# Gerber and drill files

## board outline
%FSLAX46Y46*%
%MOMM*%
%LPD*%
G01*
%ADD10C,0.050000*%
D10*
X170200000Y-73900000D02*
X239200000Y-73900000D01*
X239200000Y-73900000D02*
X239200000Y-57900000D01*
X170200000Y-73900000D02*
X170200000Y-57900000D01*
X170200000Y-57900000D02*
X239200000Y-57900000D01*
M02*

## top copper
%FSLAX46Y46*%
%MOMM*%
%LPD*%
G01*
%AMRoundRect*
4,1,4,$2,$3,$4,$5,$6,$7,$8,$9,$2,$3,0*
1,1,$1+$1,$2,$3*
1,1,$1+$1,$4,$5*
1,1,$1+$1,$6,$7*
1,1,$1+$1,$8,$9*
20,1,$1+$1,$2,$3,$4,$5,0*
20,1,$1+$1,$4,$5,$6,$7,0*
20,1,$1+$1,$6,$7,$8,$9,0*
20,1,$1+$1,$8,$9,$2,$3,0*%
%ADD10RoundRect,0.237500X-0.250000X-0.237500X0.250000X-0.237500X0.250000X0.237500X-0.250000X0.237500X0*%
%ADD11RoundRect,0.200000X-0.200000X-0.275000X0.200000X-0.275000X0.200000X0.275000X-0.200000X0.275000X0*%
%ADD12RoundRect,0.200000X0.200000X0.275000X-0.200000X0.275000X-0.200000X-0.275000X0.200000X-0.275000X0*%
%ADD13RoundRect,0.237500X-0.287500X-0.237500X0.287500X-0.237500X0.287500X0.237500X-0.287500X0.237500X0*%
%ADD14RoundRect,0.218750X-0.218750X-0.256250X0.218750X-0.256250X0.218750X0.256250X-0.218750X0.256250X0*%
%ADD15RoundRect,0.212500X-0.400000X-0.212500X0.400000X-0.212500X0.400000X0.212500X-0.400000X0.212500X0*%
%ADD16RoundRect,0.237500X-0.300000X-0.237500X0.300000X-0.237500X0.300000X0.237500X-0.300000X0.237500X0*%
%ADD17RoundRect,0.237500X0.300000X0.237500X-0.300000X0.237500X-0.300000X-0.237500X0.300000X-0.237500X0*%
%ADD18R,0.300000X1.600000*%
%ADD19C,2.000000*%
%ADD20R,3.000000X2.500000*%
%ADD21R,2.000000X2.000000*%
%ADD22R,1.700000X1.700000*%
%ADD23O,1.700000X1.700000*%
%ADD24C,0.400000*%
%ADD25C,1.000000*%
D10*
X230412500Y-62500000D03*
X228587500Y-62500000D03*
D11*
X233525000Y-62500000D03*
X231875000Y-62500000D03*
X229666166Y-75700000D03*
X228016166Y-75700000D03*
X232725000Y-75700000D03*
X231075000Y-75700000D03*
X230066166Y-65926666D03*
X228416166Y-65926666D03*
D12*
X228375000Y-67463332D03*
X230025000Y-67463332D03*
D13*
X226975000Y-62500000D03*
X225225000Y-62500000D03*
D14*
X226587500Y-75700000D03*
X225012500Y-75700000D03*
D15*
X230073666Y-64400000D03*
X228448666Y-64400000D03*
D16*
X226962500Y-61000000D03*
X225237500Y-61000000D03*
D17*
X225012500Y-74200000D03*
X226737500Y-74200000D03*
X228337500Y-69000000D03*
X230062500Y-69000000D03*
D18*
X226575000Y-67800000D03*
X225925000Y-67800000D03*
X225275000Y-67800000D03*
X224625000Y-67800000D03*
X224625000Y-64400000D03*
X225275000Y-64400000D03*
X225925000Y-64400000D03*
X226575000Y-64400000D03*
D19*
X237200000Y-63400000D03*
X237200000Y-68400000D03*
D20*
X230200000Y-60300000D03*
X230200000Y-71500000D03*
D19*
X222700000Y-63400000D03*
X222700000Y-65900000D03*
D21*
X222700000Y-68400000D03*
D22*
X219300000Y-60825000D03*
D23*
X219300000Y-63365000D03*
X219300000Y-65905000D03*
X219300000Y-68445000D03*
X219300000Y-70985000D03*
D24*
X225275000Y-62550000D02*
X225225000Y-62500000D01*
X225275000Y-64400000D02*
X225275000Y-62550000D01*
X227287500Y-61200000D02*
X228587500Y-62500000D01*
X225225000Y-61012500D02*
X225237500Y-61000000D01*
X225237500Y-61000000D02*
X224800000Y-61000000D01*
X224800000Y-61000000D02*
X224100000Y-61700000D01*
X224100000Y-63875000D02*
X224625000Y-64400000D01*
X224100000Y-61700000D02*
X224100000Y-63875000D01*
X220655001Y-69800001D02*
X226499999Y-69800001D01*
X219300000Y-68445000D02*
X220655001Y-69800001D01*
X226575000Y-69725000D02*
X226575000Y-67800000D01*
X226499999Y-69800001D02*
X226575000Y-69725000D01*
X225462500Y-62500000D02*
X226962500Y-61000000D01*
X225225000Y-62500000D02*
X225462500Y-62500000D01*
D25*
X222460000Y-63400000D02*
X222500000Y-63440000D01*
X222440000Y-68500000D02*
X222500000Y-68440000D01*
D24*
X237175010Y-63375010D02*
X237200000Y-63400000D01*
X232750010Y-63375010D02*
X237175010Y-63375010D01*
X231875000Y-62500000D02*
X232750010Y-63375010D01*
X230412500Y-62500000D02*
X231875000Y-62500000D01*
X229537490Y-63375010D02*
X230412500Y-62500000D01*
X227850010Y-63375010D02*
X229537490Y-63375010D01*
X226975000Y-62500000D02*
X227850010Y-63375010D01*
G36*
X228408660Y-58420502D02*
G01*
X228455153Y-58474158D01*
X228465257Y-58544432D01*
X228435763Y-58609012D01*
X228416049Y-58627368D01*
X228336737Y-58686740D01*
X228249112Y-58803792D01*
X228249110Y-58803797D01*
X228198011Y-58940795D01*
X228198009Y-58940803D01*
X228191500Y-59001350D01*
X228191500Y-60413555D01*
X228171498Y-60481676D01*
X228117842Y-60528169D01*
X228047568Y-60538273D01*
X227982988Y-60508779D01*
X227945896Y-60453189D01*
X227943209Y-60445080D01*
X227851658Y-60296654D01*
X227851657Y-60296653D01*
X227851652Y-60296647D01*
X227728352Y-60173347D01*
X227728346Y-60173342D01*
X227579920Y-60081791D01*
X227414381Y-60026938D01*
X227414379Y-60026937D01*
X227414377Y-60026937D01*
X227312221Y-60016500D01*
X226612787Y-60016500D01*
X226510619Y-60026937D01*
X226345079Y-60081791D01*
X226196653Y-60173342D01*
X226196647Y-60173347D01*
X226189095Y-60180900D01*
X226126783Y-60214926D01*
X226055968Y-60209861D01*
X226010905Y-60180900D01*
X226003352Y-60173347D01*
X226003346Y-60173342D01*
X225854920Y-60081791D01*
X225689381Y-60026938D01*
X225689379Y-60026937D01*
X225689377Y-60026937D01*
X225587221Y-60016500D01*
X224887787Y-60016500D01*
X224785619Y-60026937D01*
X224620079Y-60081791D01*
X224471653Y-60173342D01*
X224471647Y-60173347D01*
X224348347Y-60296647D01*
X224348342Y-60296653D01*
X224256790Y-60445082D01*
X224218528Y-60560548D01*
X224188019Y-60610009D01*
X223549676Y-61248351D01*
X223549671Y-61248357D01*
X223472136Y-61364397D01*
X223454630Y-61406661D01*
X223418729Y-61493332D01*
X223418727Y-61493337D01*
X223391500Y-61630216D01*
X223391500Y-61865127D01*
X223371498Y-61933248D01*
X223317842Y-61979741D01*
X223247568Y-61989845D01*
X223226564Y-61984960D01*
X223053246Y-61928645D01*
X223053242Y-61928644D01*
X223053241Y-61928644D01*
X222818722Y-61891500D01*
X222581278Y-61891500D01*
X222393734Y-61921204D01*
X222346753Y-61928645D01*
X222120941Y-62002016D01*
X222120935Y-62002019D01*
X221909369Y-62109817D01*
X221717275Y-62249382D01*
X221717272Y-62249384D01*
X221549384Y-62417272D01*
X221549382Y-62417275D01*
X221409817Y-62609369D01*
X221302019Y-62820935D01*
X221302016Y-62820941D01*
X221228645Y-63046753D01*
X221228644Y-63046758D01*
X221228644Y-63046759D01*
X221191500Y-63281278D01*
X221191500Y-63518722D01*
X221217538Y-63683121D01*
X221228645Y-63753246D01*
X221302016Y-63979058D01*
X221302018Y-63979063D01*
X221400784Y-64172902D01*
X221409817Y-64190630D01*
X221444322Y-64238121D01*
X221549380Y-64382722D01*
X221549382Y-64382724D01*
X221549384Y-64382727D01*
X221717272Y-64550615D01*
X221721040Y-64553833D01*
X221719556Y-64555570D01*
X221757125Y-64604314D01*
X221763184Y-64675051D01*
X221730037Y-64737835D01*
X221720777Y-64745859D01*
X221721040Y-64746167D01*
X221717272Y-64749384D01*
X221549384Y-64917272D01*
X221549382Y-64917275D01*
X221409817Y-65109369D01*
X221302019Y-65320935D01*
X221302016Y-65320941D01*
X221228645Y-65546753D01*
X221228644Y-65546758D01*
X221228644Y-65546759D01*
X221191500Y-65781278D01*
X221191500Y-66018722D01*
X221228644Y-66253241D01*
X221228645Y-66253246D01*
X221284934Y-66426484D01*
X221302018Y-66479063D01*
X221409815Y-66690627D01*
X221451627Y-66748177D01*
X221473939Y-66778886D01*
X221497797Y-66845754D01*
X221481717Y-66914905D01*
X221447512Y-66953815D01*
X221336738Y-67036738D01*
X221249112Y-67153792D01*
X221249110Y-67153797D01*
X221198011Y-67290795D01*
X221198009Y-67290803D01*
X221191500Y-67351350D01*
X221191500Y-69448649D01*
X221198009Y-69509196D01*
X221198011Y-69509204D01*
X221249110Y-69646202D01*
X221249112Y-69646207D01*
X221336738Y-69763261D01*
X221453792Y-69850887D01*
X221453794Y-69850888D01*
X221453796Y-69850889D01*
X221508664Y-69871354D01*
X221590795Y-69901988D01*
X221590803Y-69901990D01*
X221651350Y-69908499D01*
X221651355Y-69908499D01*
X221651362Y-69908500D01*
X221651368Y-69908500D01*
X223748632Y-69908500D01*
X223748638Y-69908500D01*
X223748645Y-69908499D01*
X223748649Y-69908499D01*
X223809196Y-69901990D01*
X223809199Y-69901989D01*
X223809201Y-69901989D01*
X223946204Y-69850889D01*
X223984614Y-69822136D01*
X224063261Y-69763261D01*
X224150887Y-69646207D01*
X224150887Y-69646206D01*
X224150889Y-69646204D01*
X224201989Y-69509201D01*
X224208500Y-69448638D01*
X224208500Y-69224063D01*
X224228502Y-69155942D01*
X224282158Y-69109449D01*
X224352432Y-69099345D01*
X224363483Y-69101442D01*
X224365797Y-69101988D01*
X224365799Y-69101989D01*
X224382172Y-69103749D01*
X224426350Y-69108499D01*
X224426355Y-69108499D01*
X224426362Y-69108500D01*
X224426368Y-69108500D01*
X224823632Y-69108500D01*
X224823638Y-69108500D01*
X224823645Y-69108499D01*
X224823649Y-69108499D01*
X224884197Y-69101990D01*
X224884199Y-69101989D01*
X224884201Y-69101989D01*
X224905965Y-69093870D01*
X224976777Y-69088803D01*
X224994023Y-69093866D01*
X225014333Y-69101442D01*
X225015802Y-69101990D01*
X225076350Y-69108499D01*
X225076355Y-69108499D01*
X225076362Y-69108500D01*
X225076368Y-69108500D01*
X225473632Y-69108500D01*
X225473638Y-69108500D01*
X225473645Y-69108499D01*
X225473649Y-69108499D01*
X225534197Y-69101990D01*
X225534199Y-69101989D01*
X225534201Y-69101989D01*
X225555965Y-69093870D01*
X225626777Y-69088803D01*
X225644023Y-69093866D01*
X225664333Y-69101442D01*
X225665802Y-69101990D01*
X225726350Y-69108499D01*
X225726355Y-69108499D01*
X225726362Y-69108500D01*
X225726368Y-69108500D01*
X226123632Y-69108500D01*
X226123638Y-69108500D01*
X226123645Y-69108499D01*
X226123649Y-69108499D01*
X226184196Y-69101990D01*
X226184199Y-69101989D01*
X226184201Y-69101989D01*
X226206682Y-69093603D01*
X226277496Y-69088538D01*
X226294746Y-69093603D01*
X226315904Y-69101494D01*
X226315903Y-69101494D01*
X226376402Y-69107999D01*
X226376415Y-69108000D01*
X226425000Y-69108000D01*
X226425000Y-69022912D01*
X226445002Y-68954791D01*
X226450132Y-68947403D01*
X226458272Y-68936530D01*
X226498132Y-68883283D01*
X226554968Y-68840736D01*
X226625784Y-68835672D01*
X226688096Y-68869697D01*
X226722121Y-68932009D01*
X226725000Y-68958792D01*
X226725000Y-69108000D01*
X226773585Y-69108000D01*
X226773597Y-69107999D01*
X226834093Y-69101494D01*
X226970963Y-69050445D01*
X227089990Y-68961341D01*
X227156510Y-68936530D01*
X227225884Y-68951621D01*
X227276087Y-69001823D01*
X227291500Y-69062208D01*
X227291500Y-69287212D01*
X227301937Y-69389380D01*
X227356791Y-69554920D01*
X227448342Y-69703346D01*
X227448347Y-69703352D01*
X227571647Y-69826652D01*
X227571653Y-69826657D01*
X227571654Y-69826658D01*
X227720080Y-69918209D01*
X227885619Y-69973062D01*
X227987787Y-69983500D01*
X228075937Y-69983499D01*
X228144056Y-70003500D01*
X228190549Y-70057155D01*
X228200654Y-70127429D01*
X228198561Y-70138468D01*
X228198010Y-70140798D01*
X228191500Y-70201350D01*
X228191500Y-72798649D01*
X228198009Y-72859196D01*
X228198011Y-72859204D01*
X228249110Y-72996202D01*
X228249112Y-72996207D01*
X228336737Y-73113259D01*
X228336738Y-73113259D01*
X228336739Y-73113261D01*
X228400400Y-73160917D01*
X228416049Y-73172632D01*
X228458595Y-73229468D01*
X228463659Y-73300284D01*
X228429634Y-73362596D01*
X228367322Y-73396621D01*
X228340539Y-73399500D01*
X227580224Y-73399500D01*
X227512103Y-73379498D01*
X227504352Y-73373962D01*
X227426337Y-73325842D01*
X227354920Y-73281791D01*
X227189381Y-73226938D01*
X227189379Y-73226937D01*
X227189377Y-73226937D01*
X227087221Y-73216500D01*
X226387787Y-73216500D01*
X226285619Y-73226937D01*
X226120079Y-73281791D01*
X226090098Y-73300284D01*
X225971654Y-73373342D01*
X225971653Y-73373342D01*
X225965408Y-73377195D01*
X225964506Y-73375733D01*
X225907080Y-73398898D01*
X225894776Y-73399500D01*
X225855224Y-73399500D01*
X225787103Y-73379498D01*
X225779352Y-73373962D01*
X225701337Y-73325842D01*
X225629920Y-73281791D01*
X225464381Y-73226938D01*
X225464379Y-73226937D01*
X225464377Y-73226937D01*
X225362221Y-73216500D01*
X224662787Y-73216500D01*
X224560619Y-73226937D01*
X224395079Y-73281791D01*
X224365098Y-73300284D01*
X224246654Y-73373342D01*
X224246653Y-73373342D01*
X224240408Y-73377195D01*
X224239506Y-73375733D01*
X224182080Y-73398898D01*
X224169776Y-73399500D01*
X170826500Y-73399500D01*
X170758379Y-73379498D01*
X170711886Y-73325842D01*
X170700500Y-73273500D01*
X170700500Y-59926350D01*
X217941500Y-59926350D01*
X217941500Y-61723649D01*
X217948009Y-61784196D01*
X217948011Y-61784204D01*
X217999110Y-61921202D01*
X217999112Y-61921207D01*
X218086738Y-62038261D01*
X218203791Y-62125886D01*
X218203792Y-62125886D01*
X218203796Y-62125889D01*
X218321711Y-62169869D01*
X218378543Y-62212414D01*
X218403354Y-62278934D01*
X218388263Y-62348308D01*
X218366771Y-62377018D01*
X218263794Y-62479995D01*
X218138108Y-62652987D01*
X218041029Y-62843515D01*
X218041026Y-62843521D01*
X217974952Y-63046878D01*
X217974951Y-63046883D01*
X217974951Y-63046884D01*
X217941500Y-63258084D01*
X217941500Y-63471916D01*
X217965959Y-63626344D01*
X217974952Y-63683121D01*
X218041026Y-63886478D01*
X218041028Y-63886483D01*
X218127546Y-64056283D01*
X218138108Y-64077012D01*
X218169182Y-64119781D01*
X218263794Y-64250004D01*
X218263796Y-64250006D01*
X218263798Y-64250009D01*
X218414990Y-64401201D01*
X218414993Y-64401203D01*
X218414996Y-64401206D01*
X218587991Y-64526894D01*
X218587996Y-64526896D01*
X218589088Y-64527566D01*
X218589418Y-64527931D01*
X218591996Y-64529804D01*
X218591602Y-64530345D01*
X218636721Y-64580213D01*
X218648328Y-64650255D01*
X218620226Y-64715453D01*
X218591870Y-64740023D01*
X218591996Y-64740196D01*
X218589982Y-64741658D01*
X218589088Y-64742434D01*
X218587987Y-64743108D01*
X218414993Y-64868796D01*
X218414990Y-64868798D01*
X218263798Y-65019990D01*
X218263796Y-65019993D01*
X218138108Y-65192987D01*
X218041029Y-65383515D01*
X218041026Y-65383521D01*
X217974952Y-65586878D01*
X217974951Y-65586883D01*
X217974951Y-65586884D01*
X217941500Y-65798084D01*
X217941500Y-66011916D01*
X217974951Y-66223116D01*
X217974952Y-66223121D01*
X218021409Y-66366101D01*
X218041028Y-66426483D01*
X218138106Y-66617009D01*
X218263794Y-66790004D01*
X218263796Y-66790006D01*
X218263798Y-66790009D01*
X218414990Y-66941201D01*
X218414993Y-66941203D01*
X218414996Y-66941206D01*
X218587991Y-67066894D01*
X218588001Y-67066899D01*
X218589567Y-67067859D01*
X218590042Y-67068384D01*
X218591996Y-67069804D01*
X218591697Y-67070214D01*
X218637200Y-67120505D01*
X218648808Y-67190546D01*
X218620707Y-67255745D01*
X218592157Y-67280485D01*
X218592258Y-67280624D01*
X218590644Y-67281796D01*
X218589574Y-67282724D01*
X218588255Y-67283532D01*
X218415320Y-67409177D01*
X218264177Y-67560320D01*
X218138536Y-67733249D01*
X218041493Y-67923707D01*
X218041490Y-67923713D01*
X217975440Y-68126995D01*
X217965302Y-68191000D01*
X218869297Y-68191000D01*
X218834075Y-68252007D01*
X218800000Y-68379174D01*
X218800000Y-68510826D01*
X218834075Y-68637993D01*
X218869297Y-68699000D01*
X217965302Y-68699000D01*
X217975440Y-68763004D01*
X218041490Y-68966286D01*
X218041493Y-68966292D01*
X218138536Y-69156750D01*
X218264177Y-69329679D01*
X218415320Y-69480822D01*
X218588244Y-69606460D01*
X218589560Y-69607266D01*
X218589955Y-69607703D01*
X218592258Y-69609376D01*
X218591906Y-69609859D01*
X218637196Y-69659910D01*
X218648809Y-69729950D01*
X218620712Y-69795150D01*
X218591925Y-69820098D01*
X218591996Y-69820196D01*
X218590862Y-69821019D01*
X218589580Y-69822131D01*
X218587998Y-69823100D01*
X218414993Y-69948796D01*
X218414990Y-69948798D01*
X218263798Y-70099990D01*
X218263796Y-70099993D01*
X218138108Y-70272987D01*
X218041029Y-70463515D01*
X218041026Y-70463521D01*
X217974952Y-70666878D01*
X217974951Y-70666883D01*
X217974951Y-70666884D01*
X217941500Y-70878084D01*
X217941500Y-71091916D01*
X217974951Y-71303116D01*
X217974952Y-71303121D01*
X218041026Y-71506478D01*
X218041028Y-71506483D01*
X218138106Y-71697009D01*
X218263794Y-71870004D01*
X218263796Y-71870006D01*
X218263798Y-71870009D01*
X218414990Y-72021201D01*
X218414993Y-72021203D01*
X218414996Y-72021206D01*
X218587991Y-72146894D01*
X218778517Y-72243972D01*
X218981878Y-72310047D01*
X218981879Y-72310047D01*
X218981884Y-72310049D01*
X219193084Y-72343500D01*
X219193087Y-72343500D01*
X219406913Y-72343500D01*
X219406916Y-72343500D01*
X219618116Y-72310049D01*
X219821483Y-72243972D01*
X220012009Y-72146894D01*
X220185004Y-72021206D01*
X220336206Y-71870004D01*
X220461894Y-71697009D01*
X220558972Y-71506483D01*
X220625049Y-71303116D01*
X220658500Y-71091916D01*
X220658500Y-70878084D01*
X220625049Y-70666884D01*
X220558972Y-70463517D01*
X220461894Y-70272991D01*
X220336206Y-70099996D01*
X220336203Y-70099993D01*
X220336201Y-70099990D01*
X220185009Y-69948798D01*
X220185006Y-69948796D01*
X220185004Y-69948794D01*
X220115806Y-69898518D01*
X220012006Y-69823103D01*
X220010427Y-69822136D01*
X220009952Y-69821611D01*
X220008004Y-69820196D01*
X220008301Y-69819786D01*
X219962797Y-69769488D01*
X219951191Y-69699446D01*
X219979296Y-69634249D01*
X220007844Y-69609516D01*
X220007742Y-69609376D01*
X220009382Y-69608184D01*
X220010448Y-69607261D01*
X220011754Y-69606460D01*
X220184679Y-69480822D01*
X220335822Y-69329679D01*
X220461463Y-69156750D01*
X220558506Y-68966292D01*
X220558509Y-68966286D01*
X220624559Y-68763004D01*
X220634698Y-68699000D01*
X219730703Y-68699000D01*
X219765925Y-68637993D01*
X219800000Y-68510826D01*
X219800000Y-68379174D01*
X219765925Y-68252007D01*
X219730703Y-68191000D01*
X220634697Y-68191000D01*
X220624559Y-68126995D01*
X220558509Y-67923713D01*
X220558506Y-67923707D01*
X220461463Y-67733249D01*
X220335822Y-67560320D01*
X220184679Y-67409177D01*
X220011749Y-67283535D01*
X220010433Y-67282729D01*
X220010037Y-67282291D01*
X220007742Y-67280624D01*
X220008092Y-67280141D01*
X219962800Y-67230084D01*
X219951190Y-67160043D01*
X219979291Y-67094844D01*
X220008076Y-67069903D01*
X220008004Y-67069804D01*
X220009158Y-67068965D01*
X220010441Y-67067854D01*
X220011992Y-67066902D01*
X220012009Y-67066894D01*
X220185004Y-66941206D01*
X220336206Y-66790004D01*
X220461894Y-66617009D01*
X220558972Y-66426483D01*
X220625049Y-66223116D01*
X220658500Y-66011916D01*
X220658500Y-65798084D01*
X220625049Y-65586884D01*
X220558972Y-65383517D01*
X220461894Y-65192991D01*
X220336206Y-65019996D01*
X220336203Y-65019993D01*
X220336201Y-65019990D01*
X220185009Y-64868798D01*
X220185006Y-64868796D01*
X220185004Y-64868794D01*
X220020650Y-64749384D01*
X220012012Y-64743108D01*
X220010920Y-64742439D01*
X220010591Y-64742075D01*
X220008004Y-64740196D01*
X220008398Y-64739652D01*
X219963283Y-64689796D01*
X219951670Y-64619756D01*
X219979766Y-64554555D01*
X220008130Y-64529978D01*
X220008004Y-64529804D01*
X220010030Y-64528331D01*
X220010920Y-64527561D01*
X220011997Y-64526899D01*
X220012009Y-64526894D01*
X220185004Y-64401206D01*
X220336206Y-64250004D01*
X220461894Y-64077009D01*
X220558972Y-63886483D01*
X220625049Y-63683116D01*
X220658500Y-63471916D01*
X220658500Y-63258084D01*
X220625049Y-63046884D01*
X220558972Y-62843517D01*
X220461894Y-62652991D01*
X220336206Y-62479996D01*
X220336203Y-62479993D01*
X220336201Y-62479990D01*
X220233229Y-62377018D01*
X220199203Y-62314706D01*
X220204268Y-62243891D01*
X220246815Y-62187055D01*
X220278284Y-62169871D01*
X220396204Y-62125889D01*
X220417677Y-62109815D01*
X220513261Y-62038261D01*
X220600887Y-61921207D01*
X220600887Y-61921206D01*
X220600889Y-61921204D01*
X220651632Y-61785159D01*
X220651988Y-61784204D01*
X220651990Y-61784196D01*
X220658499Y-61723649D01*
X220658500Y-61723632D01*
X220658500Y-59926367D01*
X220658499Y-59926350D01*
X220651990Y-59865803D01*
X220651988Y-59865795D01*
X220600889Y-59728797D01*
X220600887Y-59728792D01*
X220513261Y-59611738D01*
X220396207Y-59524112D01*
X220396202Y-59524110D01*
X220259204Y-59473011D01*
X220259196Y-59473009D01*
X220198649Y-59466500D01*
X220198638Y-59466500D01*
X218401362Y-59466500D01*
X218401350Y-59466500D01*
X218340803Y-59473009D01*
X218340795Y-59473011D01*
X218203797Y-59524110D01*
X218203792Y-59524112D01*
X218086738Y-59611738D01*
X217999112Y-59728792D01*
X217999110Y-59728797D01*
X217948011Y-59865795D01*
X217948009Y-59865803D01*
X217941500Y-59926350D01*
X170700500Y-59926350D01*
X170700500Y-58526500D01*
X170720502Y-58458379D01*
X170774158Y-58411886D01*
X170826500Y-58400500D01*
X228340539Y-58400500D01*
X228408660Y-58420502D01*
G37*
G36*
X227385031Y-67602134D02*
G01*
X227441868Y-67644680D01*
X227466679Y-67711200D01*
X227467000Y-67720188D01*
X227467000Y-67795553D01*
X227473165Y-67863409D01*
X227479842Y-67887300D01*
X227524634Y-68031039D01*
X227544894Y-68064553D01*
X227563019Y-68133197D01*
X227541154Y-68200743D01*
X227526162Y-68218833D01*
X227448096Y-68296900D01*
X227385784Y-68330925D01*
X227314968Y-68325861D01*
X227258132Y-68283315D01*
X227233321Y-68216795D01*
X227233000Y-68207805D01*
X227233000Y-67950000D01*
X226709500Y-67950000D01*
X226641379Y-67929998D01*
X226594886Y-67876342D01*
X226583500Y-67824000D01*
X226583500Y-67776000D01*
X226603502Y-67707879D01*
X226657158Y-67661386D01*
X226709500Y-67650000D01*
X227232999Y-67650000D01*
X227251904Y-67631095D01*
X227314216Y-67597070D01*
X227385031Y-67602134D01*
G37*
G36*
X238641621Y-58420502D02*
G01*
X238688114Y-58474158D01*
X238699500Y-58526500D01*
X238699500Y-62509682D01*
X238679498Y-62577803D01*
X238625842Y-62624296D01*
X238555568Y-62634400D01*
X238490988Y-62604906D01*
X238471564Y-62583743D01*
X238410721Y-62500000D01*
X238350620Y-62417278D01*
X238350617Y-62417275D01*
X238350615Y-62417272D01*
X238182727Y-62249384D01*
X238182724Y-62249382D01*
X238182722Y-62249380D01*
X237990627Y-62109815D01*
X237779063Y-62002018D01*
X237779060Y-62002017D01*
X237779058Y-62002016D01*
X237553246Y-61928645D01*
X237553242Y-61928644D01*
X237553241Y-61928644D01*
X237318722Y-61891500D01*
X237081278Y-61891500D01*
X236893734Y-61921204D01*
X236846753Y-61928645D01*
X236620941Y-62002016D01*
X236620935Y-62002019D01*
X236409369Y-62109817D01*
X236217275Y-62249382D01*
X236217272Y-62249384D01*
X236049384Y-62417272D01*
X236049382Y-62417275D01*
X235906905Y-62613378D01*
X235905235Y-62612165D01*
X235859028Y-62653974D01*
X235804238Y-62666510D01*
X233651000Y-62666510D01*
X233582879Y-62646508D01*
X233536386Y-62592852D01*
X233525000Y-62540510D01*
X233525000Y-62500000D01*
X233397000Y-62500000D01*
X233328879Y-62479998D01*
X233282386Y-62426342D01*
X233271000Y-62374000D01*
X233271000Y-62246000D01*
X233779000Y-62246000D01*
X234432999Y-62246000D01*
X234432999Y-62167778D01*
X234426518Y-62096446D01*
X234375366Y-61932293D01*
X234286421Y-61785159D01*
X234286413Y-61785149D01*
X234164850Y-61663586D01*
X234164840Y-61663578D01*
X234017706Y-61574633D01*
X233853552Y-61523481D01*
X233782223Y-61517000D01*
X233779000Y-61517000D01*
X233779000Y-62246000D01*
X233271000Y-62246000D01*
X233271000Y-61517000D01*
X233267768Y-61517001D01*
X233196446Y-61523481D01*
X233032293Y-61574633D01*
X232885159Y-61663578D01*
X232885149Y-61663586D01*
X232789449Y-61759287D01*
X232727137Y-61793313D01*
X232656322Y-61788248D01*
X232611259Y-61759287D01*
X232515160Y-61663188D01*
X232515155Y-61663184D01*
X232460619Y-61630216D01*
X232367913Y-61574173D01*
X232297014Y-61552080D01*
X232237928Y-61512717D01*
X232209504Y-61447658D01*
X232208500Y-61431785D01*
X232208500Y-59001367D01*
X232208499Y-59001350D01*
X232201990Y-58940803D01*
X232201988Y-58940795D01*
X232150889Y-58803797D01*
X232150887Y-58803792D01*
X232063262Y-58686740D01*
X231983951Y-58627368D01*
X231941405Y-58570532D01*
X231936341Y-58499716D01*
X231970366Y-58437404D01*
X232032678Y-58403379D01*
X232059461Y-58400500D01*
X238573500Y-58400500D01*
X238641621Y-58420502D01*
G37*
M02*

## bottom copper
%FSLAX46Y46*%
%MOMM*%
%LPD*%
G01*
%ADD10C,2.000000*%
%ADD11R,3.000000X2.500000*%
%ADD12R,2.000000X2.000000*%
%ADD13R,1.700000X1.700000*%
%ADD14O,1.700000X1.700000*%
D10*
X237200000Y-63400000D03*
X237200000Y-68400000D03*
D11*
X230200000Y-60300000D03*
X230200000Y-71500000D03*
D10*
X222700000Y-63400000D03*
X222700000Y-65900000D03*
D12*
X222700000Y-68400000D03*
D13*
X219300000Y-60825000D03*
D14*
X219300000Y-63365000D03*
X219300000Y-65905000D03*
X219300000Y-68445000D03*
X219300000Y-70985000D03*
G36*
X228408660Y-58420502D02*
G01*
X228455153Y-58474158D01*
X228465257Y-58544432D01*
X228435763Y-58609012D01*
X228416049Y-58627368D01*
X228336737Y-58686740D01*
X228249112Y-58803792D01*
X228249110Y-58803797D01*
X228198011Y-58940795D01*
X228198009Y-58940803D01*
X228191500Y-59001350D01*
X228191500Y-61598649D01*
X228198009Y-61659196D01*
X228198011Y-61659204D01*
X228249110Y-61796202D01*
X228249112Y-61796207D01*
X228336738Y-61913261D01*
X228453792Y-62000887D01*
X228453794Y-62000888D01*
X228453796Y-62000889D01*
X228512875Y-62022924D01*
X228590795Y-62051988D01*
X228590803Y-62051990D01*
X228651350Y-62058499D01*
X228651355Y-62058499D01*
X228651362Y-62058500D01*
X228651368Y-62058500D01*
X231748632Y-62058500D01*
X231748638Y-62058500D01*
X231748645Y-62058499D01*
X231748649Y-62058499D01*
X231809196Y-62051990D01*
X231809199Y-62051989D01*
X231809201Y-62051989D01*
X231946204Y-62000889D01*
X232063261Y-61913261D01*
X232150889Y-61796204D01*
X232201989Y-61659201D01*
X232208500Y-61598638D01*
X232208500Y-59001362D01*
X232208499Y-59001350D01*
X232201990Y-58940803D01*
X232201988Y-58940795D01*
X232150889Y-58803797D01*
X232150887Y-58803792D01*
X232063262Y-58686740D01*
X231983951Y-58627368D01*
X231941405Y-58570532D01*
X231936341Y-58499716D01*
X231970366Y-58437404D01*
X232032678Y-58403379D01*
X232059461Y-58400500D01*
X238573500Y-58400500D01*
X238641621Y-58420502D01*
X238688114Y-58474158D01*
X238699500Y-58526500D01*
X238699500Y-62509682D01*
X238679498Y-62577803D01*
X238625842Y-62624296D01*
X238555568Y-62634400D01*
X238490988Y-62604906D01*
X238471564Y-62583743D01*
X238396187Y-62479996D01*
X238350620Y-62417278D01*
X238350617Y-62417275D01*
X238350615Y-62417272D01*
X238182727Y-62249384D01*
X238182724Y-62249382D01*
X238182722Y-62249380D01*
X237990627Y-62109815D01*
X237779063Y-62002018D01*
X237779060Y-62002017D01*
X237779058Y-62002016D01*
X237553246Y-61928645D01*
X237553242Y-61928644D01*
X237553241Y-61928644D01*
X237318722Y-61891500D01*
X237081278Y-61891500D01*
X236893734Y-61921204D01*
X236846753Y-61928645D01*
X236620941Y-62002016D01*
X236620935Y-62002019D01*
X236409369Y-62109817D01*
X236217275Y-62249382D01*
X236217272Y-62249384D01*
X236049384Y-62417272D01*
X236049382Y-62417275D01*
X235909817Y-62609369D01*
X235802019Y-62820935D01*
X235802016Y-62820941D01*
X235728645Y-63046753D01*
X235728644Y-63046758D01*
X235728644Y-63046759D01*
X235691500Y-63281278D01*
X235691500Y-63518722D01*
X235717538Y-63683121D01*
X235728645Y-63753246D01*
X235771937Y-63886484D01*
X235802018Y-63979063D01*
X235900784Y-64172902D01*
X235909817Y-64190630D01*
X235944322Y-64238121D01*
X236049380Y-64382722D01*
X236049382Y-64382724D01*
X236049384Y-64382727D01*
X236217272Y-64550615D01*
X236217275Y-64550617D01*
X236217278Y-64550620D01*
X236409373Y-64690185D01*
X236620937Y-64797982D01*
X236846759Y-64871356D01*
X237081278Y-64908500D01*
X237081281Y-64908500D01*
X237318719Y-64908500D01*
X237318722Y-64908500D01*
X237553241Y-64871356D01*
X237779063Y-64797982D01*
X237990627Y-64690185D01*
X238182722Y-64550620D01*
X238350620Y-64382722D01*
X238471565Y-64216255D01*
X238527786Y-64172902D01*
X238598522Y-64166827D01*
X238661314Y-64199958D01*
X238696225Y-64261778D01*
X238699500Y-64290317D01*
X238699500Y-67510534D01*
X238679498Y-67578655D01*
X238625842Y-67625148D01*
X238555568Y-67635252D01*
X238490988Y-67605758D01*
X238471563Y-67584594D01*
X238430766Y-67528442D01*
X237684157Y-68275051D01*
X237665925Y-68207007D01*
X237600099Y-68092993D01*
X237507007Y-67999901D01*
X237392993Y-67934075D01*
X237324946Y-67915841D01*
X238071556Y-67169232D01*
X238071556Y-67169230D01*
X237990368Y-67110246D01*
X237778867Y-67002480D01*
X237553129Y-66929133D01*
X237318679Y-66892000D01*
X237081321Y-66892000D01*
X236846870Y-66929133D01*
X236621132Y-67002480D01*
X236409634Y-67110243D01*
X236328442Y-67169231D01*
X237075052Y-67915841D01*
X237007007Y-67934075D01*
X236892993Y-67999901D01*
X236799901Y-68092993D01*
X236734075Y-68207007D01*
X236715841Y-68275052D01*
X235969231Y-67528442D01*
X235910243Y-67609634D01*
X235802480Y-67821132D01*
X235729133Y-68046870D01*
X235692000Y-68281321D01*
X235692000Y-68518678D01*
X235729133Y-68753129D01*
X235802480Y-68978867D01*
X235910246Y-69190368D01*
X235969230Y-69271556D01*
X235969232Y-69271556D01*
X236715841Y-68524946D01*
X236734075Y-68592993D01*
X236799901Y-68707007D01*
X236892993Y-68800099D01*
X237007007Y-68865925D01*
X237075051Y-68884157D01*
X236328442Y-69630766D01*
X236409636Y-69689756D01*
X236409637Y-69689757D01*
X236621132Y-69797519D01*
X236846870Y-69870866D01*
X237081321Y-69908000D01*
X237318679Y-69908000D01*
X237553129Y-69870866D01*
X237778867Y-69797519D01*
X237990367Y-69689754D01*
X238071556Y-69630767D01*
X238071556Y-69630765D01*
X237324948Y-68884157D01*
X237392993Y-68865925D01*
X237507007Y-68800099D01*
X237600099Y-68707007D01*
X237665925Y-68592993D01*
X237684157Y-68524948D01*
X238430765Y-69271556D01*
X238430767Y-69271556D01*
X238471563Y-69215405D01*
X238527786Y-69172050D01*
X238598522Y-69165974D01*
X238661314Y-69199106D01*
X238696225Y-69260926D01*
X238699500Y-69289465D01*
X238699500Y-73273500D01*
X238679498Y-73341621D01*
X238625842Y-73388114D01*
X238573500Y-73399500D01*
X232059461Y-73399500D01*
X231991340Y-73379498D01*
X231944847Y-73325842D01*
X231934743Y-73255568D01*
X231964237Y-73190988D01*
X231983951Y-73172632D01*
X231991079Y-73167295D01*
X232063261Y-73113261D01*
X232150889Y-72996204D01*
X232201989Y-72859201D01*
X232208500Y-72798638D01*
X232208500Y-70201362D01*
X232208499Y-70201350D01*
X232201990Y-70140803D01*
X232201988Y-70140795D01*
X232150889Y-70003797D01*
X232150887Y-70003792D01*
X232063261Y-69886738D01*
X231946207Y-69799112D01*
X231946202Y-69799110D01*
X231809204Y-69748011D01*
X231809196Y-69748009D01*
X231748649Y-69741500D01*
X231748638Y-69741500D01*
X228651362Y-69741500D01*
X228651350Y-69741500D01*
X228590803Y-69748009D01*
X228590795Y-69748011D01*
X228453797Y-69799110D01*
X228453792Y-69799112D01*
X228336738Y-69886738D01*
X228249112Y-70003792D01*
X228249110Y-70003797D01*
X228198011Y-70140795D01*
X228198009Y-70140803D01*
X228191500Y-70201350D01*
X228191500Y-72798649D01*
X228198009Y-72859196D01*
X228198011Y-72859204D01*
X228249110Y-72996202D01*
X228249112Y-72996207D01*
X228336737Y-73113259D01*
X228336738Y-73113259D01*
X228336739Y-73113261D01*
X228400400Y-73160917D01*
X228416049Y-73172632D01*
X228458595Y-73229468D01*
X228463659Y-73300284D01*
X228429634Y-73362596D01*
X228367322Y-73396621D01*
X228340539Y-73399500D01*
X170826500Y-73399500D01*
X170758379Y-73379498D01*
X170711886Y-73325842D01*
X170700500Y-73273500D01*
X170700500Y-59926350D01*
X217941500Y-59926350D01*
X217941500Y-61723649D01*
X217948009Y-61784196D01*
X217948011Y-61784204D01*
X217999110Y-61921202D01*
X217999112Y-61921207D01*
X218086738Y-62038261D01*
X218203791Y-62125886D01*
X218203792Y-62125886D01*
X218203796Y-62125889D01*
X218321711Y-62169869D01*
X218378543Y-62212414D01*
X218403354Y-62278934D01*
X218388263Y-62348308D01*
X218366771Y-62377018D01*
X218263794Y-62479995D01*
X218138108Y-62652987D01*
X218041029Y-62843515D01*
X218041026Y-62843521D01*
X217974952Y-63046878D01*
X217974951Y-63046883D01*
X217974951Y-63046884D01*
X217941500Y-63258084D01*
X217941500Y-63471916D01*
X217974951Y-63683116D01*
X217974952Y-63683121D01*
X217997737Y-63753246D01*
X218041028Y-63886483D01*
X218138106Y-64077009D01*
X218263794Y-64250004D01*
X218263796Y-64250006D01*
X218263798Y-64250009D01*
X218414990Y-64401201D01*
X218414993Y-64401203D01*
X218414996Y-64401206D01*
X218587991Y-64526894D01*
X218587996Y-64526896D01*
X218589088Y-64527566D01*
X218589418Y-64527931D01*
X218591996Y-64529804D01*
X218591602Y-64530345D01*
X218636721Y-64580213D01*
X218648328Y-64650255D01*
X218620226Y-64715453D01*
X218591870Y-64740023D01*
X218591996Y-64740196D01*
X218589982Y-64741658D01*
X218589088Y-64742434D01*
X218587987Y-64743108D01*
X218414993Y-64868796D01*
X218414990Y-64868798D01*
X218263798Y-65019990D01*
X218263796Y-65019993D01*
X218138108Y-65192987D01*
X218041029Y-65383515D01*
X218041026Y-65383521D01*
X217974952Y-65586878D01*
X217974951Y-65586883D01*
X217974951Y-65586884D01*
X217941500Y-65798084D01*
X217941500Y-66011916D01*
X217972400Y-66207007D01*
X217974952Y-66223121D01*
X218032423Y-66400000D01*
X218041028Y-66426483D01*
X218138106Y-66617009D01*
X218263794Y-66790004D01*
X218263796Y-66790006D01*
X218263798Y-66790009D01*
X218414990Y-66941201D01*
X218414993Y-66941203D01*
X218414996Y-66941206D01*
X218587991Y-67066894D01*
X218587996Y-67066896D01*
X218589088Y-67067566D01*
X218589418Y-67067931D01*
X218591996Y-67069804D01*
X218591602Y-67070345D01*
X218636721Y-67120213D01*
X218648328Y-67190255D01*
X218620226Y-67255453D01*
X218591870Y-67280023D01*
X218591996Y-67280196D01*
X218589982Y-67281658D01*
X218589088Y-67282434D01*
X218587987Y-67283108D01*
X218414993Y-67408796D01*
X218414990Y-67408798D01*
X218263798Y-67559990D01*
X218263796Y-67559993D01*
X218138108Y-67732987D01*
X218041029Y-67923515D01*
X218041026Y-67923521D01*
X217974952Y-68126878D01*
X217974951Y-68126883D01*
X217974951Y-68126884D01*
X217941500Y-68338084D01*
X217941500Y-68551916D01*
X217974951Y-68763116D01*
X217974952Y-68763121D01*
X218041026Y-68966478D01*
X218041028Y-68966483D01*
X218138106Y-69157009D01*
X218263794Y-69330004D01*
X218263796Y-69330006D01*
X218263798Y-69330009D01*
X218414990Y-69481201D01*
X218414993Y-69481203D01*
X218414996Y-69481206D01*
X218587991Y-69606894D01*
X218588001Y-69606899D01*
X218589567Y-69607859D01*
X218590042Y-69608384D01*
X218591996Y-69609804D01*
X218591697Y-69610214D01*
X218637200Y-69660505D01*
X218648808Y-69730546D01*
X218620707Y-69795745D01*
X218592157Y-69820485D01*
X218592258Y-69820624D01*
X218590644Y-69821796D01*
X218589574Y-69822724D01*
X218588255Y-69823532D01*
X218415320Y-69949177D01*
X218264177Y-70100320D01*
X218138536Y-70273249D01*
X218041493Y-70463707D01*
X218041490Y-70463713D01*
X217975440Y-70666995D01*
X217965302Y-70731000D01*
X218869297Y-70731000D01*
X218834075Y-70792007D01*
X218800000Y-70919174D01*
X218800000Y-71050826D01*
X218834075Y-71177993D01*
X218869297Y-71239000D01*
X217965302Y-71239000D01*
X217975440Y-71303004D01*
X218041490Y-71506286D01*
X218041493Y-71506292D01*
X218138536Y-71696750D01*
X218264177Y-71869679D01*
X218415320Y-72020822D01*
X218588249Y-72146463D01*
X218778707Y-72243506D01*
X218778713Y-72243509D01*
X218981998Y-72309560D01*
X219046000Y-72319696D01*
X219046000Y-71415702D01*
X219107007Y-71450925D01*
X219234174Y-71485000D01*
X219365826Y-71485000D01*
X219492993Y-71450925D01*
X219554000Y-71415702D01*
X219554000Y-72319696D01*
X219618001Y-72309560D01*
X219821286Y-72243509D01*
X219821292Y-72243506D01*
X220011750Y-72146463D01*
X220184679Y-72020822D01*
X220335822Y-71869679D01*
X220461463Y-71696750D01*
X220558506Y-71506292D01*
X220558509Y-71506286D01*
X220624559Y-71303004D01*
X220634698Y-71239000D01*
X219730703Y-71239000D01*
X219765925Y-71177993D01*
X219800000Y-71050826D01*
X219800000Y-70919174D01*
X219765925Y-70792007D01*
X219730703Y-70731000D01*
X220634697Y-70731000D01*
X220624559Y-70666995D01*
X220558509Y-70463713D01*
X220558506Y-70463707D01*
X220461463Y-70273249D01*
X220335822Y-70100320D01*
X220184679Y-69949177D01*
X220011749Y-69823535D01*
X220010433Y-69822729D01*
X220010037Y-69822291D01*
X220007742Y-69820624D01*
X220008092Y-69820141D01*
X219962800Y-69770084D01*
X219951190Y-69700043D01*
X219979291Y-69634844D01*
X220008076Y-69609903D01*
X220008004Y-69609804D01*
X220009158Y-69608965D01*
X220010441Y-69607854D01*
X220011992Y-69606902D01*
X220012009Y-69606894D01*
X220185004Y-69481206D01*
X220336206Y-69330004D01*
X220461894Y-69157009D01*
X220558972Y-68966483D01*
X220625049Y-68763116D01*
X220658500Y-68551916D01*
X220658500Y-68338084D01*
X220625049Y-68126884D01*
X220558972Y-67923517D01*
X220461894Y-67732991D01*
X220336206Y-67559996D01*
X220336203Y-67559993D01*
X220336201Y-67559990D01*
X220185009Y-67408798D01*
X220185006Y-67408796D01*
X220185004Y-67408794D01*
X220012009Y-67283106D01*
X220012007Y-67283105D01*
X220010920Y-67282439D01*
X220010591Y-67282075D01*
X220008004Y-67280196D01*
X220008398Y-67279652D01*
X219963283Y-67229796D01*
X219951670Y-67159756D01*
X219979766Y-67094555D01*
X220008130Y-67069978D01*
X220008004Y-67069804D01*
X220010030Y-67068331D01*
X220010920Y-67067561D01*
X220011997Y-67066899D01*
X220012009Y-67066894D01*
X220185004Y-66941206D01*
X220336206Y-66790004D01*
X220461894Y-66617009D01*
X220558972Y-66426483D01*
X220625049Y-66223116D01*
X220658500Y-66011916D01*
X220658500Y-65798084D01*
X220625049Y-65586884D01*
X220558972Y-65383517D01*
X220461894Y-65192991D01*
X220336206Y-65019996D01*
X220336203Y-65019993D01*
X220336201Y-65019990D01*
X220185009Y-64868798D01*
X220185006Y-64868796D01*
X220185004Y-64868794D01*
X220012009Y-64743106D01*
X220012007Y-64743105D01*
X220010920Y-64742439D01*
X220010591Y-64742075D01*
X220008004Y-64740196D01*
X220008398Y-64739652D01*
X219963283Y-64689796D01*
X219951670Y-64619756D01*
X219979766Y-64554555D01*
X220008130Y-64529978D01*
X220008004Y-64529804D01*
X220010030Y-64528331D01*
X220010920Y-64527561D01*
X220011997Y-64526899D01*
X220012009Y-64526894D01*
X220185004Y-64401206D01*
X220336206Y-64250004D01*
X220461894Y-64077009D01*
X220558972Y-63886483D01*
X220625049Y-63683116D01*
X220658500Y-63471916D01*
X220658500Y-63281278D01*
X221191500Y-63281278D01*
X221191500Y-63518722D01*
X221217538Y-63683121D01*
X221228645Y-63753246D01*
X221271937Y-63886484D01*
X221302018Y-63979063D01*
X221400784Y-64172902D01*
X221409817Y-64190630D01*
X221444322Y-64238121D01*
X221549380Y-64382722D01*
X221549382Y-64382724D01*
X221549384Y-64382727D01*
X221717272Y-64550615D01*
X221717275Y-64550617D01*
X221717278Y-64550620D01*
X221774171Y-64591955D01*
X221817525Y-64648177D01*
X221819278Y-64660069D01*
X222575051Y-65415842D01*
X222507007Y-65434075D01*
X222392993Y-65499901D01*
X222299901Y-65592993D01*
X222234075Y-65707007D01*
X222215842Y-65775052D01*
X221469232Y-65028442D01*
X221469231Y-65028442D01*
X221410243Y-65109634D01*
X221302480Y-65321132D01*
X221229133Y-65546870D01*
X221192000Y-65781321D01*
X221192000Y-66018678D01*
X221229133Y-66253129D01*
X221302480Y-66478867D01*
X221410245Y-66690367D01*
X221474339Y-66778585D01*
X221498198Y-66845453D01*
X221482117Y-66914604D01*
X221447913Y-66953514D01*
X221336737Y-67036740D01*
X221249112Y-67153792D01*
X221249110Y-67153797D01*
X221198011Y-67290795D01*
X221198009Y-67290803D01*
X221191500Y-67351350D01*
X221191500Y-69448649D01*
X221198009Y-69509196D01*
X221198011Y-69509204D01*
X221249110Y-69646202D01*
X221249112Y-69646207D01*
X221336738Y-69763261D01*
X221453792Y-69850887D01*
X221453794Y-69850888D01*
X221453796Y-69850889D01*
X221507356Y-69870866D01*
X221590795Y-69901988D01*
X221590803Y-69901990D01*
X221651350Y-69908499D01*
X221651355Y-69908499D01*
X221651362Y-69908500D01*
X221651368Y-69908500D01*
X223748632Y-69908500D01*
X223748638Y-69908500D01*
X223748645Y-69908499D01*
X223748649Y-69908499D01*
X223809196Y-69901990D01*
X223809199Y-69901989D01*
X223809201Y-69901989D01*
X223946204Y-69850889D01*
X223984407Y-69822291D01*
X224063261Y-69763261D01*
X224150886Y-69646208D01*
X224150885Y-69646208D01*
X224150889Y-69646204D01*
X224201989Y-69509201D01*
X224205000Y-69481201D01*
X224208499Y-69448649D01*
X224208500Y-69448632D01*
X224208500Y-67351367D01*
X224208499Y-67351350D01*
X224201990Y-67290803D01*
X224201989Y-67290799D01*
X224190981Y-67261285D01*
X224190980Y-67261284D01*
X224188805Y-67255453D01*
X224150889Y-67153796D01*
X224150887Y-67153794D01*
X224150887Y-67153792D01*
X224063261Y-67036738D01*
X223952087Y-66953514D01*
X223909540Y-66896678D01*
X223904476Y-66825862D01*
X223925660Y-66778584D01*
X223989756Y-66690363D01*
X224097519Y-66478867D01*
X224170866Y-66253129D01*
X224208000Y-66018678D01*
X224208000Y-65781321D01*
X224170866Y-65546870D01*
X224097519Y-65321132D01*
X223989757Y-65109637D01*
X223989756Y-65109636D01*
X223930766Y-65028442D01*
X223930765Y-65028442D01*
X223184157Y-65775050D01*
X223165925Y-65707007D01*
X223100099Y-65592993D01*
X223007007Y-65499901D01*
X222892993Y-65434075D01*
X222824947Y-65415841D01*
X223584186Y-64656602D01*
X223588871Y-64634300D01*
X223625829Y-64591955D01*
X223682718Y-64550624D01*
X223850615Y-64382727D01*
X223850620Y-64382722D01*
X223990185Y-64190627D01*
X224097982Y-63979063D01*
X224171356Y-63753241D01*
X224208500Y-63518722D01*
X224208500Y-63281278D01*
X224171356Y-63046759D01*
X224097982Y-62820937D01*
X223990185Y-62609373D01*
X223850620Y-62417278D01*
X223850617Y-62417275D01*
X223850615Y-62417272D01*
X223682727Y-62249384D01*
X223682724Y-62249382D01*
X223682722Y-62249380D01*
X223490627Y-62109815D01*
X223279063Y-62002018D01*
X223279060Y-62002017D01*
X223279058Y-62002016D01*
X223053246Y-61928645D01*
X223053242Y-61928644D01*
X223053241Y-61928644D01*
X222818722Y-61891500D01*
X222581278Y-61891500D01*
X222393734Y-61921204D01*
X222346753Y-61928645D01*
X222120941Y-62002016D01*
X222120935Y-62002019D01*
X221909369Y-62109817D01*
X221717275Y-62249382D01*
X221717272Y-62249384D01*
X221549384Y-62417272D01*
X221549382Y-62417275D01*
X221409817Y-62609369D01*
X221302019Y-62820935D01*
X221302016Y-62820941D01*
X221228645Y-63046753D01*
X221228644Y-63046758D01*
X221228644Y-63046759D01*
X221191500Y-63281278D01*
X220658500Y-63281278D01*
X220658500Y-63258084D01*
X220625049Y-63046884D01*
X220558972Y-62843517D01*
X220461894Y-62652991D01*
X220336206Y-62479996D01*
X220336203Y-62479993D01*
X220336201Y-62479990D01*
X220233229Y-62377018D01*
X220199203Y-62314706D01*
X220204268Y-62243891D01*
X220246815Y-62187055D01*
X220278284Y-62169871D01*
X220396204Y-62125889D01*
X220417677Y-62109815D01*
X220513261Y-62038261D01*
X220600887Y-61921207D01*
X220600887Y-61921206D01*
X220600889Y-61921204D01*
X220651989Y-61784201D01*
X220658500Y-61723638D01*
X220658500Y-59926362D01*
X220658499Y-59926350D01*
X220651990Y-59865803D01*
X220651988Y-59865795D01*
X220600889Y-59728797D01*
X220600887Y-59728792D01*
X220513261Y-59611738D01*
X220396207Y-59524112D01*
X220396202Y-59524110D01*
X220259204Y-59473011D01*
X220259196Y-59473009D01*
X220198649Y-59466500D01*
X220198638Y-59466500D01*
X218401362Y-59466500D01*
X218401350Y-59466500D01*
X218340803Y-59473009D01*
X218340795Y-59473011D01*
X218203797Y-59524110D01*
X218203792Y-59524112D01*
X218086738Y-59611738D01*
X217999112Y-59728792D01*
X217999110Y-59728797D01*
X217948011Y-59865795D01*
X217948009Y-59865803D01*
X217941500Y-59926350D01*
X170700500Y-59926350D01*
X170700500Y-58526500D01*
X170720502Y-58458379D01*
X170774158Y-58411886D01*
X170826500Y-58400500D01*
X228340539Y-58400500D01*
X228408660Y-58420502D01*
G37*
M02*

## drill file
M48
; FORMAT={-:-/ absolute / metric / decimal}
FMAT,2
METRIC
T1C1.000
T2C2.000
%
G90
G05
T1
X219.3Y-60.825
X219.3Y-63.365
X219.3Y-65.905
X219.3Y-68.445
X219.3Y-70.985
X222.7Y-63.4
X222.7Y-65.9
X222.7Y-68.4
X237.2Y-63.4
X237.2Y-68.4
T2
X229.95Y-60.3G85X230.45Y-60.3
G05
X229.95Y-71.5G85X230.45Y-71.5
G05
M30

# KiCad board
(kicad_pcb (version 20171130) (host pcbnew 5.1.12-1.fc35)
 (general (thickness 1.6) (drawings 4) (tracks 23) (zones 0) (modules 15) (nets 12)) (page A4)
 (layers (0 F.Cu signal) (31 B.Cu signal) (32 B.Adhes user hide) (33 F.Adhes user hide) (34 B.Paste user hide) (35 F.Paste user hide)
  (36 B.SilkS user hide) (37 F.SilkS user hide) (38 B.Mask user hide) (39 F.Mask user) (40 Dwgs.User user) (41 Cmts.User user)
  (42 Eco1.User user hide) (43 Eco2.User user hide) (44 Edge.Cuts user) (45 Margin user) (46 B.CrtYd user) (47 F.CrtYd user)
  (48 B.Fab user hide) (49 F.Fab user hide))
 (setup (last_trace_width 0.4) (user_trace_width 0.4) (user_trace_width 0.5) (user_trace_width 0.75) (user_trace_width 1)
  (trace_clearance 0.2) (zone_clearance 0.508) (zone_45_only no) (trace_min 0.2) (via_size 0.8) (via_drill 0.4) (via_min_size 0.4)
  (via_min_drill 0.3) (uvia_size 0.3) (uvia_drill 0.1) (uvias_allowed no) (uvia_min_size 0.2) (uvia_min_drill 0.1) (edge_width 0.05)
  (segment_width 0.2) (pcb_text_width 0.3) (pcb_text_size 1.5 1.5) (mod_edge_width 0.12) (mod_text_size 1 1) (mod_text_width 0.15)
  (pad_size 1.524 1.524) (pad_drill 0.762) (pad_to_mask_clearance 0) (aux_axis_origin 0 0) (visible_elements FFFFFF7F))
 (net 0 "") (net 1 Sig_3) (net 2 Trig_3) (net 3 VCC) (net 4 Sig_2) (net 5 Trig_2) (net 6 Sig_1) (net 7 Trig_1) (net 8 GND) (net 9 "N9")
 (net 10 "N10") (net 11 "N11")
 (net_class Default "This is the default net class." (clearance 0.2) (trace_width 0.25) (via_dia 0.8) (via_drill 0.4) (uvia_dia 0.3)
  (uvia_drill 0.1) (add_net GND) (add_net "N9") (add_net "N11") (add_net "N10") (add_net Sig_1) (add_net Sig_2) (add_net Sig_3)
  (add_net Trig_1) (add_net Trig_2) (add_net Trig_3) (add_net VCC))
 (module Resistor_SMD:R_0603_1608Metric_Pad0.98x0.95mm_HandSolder (layer F.Cu) (at 229.5 62.5)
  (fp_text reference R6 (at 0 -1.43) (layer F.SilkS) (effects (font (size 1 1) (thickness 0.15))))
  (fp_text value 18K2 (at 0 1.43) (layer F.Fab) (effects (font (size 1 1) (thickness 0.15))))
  (pad 2 smd roundrect (at 0.9125 0) (size 0.975 0.95) (layers F.Cu F.Paste F.Mask) (roundrect_rratio 0.25) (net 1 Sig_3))
  (pad 1 smd roundrect (at -0.9125 0) (size 0.975 0.95) (layers F.Cu F.Paste F.Mask) (roundrect_rratio 0.25) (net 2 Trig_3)))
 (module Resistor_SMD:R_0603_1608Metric (layer F.Cu) (at 232.7 62.5)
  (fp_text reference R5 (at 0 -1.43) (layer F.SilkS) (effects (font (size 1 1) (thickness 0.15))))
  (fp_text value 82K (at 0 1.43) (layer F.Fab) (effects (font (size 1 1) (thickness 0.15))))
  (pad 2 smd roundrect (at 0.825 0) (size 0.8 0.95) (layers F.Cu F.Paste F.Mask) (roundrect_rratio 0.25) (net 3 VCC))
  (pad 1 smd roundrect (at -0.825 0) (size 0.8 0.95) (layers F.Cu F.Paste F.Mask) (roundrect_rratio 0.25) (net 1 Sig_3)))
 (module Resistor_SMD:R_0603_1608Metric (layer F.Cu) (at 228.841166 75.7)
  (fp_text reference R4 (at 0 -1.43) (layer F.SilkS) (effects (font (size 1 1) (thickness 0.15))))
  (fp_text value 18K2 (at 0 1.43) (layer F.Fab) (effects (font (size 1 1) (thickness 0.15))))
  (pad 2 smd roundrect (at 0.825 0) (size 0.8 0.95) (layers F.Cu F.Paste F.Mask) (roundrect_rratio 0.25) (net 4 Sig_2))
  (pad 1 smd roundrect (at -0.825 0) (size 0.8 0.95) (layers F.Cu F.Paste F.Mask) (roundrect_rratio 0.25) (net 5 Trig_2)))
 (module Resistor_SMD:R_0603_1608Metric (layer F.Cu) (at 231.9 75.7)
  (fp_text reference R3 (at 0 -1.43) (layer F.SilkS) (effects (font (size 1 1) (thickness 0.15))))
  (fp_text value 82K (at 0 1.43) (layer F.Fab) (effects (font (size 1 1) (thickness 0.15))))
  (pad 2 smd roundrect (at 0.825 0) (size 0.8 0.95) (layers F.Cu F.Paste F.Mask) (roundrect_rratio 0.25) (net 3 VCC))
  (pad 1 smd roundrect (at -0.825 0) (size 0.8 0.95) (layers F.Cu F.Paste F.Mask) (roundrect_rratio 0.25) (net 4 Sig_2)))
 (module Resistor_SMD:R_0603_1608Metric (layer F.Cu) (at 229.241166 65.926666)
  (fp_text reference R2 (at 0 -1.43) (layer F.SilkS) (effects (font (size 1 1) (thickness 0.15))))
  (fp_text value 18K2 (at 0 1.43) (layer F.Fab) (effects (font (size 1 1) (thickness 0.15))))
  (pad 2 smd roundrect (at 0.825 0) (size 0.8 0.95) (layers F.Cu F.Paste F.Mask) (roundrect_rratio 0.25) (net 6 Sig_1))
  (pad 1 smd roundrect (at -0.825 0) (size 0.8 0.95) (layers F.Cu F.Paste F.Mask) (roundrect_rratio 0.25) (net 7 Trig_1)))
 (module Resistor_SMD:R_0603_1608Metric (layer F.Cu) (at 229.2 67.463332 180)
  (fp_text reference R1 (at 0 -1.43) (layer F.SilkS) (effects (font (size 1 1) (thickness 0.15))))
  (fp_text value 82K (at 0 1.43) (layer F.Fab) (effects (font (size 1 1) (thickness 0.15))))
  (pad 2 smd roundrect (at 0.825 0 180) (size 0.8 0.95) (layers F.Cu F.Paste F.Mask) (roundrect_rratio 0.25) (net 3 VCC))
  (pad 1 smd roundrect (at -0.825 0 180) (size 0.8 0.95) (layers F.Cu F.Paste F.Mask) (roundrect_rratio 0.25) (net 6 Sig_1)))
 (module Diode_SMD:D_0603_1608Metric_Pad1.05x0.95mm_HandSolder (layer F.Cu) (at 226.1 62.5)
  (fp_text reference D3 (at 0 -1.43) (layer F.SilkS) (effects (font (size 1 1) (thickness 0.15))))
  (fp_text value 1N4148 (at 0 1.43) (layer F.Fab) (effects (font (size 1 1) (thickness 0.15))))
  (pad 2 smd roundrect (at 0.875 0) (size 1.05 0.95) (layers F.Cu F.Paste F.Mask) (roundrect_rratio 0.25) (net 1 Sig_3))
  (pad 1 smd roundrect (at -0.875 0) (size 1.05 0.95) (layers F.Cu F.Paste F.Mask) (roundrect_rratio 0.25) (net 2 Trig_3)))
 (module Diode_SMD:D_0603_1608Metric (layer F.Cu) (at 225.8 75.7)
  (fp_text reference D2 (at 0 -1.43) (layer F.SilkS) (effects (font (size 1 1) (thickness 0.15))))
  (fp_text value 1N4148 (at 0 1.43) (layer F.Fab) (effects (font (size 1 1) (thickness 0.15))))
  (pad 2 smd roundrect (at 0.7875 0) (size 0.875 0.95) (layers F.Cu F.Paste F.Mask) (roundrect_rratio 0.25) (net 4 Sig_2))
  (pad 1 smd roundrect (at -0.7875 0) (size 0.875 0.95) (layers F.Cu F.Paste F.Mask) (roundrect_rratio 0.25) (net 5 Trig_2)))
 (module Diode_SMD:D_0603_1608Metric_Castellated (layer F.Cu) (at 229.261166 64.4)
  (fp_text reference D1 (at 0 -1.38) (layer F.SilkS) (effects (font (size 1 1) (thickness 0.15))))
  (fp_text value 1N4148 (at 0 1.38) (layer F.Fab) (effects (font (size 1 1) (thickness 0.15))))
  (pad 2 smd roundrect (at 0.8125 0) (size 1.225 0.85) (layers F.Cu F.Paste F.Mask) (roundrect_rratio 0.25) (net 6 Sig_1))
  (pad 1 smd roundrect (at -0.8125 0) (size 1.225 0.85) (layers F.Cu F.Paste F.Mask) (roundrect_rratio 0.25) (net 7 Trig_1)))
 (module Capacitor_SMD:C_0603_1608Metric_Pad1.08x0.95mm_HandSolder (layer F.Cu) (at 226.1 61)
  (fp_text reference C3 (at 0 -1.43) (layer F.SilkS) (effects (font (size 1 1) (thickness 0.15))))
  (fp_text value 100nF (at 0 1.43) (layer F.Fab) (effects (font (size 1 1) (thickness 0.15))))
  (pad 2 smd roundrect (at 0.8625 0) (size 1.075 0.95) (layers F.Cu F.Paste F.Mask) (roundrect_rratio 0.25) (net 2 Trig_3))
  (pad 1 smd roundrect (at -0.8625 0) (size 1.075 0.95) (layers F.Cu F.Paste F.Mask) (roundrect_rratio 0.25) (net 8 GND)))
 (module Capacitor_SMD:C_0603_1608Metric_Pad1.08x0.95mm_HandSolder (layer F.Cu) (at 225.875 74.2 180)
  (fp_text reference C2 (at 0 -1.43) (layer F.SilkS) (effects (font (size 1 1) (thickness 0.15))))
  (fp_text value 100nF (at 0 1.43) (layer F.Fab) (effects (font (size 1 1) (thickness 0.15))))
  (pad 2 smd roundrect (at 0.8625 0 180) (size 1.075 0.95) (layers F.Cu F.Paste F.Mask) (roundrect_rratio 0.25) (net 5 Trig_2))
  (pad 1 smd roundrect (at -0.8625 0 180) (size 1.075 0.95) (layers F.Cu F.Paste F.Mask) (roundrect_rratio 0.25) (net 8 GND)))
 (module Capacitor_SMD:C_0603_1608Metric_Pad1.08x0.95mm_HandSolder (layer F.Cu) (at 229.2 69 180)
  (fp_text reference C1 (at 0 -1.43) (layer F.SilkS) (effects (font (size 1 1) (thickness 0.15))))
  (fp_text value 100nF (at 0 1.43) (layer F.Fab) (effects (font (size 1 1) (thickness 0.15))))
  (pad 2 smd roundrect (at 0.8625 0 180) (size 1.075 0.95) (layers F.Cu F.Paste F.Mask) (roundrect_rratio 0.25) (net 7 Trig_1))
  (pad 1 smd roundrect (at -0.8625 0 180) (size 1.075 0.95) (layers F.Cu F.Paste F.Mask) (roundrect_rratio 0.25) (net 8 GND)))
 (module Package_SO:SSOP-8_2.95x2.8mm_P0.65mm (layer F.Cu) (at 225.6 66.1 270)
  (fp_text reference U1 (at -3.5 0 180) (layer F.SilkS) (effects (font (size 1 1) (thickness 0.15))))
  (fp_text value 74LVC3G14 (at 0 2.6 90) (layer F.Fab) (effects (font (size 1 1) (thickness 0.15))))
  (pad 8 smd rect (at 1.7 -0.975 180) (size 0.3 1.6) (layers F.Cu F.Paste F.Mask) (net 3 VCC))
  (pad 7 smd rect (at 1.7 -0.325 180) (size 0.3 1.6) (layers F.Cu F.Paste F.Mask) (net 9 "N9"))
  (pad 6 smd rect (at 1.7 0.325 180) (size 0.3 1.6) (layers F.Cu F.Paste F.Mask) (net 5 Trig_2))
  (pad 5 smd rect (at 1.7 0.975 180) (size 0.3 1.6) (layers F.Cu F.Paste F.Mask) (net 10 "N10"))
  (pad 4 smd rect (at -1.7 0.975 180) (size 0.3 1.6) (layers F.Cu F.Paste F.Mask) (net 8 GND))
  (pad 3 smd rect (at -1.7 0.325 180) (size 0.3 1.6) (layers F.Cu F.Paste F.Mask) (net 2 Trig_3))
  (pad 2 smd rect (at -1.7 -0.325 180) (size 0.3 1.6) (layers F.Cu F.Paste F.Mask) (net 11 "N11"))
  (pad 1 smd rect (at -1.7 -0.975 180) (size 0.3 1.6) (layers F.Cu F.Paste F.Mask) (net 7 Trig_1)))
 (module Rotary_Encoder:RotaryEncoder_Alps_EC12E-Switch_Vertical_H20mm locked (layer B.Cu) (at 222.7 68.4)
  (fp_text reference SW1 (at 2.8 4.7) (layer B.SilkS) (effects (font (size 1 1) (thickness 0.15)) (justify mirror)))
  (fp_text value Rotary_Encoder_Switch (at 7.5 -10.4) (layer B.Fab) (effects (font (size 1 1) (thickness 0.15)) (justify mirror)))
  (pad S2 thru_hole circle (at 14.5 -5) (size 2 2) (drill 1) (layers *.Cu *.Mask) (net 1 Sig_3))
  (pad S1 thru_hole circle (at 14.5 0) (size 2 2) (drill 1) (layers *.Cu *.Mask) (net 8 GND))
  (pad MP thru_hole rect (at 7.5 -8.1) (size 3 2.5) (drill oval 2.5 2) (layers *.Cu *.Mask))
  (pad MP thru_hole rect (at 7.5 3.1) (size 3 2.5) (drill oval 2.5 2) (layers *.Cu *.Mask))
  (pad B thru_hole circle (at 0 -5) (size 2 2) (drill 1) (layers *.Cu *.Mask) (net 4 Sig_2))
  (pad C thru_hole circle (at 0 -2.5) (size 2 2) (drill 1) (layers *.Cu *.Mask) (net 8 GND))
  (pad A thru_hole rect (at 0 0) (size 2 2) (drill 1) (layers *.Cu *.Mask) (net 6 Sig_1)))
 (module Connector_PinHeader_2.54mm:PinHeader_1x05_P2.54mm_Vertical (layer F.Cu) (at 219.3 60.825)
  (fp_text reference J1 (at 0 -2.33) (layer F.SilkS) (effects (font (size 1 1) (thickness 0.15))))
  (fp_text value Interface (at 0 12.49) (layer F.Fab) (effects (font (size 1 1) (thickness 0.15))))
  (pad 1 thru_hole rect (at 0 0) (size 1.7 1.7) (drill 1) (layers *.Cu *.Mask) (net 9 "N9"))
  (pad 2 thru_hole oval (at 0 2.54) (size 1.7 1.7) (drill 1) (layers *.Cu *.Mask) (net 11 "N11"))
  (pad 3 thru_hole oval (at 0 5.08) (size 1.7 1.7) (drill 1) (layers *.Cu *.Mask) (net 10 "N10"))
  (pad 4 thru_hole oval (at 0 7.62) (size 1.7 1.7) (drill 1) (layers *.Cu *.Mask) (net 3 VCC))
  (pad 5 thru_hole oval (at 0 10.16) (size 1.7 1.7) (drill 1) (layers *.Cu *.Mask) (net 8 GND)))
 (gr_line (start 170.2 73.9) (end 239.2 73.9) (layer Edge.Cuts) (width 0.05))
 (gr_line (start 239.2 73.9) (end 239.2 57.9) (layer Edge.Cuts) (width 0.05))
 (gr_line (start 170.2 73.9) (end 170.2 57.9) (layer Edge.Cuts) (width 0.05))
 (gr_line (start 170.2 57.9) (end 239.2 57.9) (layer Edge.Cuts) (width 0.05))
 (segment (start 225.275 62.55) (end 225.225 62.5) (width 0.4) (layer F.Cu) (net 2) (status 30))
 (segment (start 225.275 64.4) (end 225.275 62.55) (width 0.4) (layer F.Cu) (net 2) (status 30))
 (segment (start 227.2875 61.2) (end 228.5875 62.5) (width 0.4) (layer F.Cu) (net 2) (status 30))
 (segment (start 225.225 61.0125) (end 225.2375 61) (width 0.4) (layer F.Cu) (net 8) (status 30))
 (segment (start 225.2375 61) (end 224.8 61) (width 0.4) (layer F.Cu) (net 8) (status 30))
 (segment (start 224.8 61) (end 224.1 61.7) (width 0.4) (layer F.Cu) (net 8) (status 10))
 (segment (start 224.1 63.875) (end 224.625 64.4) (width 0.4) (layer F.Cu) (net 8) (status 20))
 (segment (start 224.1 61.7) (end 224.1 63.875) (width 0.4) (layer F.Cu) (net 8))
 (segment (start 220.655001 69.800001) (end 226.499999 69.800001) (width 0.4) (layer F.Cu) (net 3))
 (segment (start 219.3 68.445) (end 220.655001 69.800001) (width 0.4) (layer F.Cu) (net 3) (status 10))
 (segment (start 226.575 69.725) (end 226.575 67.8) (width 0.4) (layer F.Cu) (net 3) (status 20))
 (segment (start 226.499999 69.800001) (end 226.575 69.725) (width 0.4) (layer F.Cu) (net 3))
 (segment (start 225.4625 62.5) (end 226.9625 61) (width 0.4) (layer F.Cu) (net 2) (status 30))
 (segment (start 225.225 62.5) (end 225.4625 62.5) (width 0.4) (layer F.Cu) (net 2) (status 30))
 (segment (start 222.46 63.4) (end 222.5 63.44) (width 1) (layer F.Cu) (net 4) (status 30))
 (segment (start 222.44 68.5) (end 222.5 68.44) (width 1) (layer F.Cu) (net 6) (status 30))
 (segment (start 237.17501 63.37501) (end 237.2 63.4) (width 0.4) (layer F.Cu) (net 1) (status 30))
 (segment (start 232.75001 63.37501) (end 237.17501 63.37501) (width 0.4) (layer F.Cu) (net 1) (status 20))
 (segment (start 231.875 62.5) (end 232.75001 63.37501) (width 0.4) (layer F.Cu) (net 1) (status 10))
 (segment (start 230.4125 62.5) (end 231.875 62.5) (width 0.4) (layer F.Cu) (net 1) (status 30))
 (segment (start 229.53749 63.37501) (end 230.4125 62.5) (width 0.4) (layer F.Cu) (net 1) (status 20))
 (segment (start 227.85001 63.37501) (end 229.53749 63.37501) (width 0.4) (layer F.Cu) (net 1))
 (segment (start 226.975 62.5) (end 227.85001 63.37501) (width 0.4) (layer F.Cu) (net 1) (status 10))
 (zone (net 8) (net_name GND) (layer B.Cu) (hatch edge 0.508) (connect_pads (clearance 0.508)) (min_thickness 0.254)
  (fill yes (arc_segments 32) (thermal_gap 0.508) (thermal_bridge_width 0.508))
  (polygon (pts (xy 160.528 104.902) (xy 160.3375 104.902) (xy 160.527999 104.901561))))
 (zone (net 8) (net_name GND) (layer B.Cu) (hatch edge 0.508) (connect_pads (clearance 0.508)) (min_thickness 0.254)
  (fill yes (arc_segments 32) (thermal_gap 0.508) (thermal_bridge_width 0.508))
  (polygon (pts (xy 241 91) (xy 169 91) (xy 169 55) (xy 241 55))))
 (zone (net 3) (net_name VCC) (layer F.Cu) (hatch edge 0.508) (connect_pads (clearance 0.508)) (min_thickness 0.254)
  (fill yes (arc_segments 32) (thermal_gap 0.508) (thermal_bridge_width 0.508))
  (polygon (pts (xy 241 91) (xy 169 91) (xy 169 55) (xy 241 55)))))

